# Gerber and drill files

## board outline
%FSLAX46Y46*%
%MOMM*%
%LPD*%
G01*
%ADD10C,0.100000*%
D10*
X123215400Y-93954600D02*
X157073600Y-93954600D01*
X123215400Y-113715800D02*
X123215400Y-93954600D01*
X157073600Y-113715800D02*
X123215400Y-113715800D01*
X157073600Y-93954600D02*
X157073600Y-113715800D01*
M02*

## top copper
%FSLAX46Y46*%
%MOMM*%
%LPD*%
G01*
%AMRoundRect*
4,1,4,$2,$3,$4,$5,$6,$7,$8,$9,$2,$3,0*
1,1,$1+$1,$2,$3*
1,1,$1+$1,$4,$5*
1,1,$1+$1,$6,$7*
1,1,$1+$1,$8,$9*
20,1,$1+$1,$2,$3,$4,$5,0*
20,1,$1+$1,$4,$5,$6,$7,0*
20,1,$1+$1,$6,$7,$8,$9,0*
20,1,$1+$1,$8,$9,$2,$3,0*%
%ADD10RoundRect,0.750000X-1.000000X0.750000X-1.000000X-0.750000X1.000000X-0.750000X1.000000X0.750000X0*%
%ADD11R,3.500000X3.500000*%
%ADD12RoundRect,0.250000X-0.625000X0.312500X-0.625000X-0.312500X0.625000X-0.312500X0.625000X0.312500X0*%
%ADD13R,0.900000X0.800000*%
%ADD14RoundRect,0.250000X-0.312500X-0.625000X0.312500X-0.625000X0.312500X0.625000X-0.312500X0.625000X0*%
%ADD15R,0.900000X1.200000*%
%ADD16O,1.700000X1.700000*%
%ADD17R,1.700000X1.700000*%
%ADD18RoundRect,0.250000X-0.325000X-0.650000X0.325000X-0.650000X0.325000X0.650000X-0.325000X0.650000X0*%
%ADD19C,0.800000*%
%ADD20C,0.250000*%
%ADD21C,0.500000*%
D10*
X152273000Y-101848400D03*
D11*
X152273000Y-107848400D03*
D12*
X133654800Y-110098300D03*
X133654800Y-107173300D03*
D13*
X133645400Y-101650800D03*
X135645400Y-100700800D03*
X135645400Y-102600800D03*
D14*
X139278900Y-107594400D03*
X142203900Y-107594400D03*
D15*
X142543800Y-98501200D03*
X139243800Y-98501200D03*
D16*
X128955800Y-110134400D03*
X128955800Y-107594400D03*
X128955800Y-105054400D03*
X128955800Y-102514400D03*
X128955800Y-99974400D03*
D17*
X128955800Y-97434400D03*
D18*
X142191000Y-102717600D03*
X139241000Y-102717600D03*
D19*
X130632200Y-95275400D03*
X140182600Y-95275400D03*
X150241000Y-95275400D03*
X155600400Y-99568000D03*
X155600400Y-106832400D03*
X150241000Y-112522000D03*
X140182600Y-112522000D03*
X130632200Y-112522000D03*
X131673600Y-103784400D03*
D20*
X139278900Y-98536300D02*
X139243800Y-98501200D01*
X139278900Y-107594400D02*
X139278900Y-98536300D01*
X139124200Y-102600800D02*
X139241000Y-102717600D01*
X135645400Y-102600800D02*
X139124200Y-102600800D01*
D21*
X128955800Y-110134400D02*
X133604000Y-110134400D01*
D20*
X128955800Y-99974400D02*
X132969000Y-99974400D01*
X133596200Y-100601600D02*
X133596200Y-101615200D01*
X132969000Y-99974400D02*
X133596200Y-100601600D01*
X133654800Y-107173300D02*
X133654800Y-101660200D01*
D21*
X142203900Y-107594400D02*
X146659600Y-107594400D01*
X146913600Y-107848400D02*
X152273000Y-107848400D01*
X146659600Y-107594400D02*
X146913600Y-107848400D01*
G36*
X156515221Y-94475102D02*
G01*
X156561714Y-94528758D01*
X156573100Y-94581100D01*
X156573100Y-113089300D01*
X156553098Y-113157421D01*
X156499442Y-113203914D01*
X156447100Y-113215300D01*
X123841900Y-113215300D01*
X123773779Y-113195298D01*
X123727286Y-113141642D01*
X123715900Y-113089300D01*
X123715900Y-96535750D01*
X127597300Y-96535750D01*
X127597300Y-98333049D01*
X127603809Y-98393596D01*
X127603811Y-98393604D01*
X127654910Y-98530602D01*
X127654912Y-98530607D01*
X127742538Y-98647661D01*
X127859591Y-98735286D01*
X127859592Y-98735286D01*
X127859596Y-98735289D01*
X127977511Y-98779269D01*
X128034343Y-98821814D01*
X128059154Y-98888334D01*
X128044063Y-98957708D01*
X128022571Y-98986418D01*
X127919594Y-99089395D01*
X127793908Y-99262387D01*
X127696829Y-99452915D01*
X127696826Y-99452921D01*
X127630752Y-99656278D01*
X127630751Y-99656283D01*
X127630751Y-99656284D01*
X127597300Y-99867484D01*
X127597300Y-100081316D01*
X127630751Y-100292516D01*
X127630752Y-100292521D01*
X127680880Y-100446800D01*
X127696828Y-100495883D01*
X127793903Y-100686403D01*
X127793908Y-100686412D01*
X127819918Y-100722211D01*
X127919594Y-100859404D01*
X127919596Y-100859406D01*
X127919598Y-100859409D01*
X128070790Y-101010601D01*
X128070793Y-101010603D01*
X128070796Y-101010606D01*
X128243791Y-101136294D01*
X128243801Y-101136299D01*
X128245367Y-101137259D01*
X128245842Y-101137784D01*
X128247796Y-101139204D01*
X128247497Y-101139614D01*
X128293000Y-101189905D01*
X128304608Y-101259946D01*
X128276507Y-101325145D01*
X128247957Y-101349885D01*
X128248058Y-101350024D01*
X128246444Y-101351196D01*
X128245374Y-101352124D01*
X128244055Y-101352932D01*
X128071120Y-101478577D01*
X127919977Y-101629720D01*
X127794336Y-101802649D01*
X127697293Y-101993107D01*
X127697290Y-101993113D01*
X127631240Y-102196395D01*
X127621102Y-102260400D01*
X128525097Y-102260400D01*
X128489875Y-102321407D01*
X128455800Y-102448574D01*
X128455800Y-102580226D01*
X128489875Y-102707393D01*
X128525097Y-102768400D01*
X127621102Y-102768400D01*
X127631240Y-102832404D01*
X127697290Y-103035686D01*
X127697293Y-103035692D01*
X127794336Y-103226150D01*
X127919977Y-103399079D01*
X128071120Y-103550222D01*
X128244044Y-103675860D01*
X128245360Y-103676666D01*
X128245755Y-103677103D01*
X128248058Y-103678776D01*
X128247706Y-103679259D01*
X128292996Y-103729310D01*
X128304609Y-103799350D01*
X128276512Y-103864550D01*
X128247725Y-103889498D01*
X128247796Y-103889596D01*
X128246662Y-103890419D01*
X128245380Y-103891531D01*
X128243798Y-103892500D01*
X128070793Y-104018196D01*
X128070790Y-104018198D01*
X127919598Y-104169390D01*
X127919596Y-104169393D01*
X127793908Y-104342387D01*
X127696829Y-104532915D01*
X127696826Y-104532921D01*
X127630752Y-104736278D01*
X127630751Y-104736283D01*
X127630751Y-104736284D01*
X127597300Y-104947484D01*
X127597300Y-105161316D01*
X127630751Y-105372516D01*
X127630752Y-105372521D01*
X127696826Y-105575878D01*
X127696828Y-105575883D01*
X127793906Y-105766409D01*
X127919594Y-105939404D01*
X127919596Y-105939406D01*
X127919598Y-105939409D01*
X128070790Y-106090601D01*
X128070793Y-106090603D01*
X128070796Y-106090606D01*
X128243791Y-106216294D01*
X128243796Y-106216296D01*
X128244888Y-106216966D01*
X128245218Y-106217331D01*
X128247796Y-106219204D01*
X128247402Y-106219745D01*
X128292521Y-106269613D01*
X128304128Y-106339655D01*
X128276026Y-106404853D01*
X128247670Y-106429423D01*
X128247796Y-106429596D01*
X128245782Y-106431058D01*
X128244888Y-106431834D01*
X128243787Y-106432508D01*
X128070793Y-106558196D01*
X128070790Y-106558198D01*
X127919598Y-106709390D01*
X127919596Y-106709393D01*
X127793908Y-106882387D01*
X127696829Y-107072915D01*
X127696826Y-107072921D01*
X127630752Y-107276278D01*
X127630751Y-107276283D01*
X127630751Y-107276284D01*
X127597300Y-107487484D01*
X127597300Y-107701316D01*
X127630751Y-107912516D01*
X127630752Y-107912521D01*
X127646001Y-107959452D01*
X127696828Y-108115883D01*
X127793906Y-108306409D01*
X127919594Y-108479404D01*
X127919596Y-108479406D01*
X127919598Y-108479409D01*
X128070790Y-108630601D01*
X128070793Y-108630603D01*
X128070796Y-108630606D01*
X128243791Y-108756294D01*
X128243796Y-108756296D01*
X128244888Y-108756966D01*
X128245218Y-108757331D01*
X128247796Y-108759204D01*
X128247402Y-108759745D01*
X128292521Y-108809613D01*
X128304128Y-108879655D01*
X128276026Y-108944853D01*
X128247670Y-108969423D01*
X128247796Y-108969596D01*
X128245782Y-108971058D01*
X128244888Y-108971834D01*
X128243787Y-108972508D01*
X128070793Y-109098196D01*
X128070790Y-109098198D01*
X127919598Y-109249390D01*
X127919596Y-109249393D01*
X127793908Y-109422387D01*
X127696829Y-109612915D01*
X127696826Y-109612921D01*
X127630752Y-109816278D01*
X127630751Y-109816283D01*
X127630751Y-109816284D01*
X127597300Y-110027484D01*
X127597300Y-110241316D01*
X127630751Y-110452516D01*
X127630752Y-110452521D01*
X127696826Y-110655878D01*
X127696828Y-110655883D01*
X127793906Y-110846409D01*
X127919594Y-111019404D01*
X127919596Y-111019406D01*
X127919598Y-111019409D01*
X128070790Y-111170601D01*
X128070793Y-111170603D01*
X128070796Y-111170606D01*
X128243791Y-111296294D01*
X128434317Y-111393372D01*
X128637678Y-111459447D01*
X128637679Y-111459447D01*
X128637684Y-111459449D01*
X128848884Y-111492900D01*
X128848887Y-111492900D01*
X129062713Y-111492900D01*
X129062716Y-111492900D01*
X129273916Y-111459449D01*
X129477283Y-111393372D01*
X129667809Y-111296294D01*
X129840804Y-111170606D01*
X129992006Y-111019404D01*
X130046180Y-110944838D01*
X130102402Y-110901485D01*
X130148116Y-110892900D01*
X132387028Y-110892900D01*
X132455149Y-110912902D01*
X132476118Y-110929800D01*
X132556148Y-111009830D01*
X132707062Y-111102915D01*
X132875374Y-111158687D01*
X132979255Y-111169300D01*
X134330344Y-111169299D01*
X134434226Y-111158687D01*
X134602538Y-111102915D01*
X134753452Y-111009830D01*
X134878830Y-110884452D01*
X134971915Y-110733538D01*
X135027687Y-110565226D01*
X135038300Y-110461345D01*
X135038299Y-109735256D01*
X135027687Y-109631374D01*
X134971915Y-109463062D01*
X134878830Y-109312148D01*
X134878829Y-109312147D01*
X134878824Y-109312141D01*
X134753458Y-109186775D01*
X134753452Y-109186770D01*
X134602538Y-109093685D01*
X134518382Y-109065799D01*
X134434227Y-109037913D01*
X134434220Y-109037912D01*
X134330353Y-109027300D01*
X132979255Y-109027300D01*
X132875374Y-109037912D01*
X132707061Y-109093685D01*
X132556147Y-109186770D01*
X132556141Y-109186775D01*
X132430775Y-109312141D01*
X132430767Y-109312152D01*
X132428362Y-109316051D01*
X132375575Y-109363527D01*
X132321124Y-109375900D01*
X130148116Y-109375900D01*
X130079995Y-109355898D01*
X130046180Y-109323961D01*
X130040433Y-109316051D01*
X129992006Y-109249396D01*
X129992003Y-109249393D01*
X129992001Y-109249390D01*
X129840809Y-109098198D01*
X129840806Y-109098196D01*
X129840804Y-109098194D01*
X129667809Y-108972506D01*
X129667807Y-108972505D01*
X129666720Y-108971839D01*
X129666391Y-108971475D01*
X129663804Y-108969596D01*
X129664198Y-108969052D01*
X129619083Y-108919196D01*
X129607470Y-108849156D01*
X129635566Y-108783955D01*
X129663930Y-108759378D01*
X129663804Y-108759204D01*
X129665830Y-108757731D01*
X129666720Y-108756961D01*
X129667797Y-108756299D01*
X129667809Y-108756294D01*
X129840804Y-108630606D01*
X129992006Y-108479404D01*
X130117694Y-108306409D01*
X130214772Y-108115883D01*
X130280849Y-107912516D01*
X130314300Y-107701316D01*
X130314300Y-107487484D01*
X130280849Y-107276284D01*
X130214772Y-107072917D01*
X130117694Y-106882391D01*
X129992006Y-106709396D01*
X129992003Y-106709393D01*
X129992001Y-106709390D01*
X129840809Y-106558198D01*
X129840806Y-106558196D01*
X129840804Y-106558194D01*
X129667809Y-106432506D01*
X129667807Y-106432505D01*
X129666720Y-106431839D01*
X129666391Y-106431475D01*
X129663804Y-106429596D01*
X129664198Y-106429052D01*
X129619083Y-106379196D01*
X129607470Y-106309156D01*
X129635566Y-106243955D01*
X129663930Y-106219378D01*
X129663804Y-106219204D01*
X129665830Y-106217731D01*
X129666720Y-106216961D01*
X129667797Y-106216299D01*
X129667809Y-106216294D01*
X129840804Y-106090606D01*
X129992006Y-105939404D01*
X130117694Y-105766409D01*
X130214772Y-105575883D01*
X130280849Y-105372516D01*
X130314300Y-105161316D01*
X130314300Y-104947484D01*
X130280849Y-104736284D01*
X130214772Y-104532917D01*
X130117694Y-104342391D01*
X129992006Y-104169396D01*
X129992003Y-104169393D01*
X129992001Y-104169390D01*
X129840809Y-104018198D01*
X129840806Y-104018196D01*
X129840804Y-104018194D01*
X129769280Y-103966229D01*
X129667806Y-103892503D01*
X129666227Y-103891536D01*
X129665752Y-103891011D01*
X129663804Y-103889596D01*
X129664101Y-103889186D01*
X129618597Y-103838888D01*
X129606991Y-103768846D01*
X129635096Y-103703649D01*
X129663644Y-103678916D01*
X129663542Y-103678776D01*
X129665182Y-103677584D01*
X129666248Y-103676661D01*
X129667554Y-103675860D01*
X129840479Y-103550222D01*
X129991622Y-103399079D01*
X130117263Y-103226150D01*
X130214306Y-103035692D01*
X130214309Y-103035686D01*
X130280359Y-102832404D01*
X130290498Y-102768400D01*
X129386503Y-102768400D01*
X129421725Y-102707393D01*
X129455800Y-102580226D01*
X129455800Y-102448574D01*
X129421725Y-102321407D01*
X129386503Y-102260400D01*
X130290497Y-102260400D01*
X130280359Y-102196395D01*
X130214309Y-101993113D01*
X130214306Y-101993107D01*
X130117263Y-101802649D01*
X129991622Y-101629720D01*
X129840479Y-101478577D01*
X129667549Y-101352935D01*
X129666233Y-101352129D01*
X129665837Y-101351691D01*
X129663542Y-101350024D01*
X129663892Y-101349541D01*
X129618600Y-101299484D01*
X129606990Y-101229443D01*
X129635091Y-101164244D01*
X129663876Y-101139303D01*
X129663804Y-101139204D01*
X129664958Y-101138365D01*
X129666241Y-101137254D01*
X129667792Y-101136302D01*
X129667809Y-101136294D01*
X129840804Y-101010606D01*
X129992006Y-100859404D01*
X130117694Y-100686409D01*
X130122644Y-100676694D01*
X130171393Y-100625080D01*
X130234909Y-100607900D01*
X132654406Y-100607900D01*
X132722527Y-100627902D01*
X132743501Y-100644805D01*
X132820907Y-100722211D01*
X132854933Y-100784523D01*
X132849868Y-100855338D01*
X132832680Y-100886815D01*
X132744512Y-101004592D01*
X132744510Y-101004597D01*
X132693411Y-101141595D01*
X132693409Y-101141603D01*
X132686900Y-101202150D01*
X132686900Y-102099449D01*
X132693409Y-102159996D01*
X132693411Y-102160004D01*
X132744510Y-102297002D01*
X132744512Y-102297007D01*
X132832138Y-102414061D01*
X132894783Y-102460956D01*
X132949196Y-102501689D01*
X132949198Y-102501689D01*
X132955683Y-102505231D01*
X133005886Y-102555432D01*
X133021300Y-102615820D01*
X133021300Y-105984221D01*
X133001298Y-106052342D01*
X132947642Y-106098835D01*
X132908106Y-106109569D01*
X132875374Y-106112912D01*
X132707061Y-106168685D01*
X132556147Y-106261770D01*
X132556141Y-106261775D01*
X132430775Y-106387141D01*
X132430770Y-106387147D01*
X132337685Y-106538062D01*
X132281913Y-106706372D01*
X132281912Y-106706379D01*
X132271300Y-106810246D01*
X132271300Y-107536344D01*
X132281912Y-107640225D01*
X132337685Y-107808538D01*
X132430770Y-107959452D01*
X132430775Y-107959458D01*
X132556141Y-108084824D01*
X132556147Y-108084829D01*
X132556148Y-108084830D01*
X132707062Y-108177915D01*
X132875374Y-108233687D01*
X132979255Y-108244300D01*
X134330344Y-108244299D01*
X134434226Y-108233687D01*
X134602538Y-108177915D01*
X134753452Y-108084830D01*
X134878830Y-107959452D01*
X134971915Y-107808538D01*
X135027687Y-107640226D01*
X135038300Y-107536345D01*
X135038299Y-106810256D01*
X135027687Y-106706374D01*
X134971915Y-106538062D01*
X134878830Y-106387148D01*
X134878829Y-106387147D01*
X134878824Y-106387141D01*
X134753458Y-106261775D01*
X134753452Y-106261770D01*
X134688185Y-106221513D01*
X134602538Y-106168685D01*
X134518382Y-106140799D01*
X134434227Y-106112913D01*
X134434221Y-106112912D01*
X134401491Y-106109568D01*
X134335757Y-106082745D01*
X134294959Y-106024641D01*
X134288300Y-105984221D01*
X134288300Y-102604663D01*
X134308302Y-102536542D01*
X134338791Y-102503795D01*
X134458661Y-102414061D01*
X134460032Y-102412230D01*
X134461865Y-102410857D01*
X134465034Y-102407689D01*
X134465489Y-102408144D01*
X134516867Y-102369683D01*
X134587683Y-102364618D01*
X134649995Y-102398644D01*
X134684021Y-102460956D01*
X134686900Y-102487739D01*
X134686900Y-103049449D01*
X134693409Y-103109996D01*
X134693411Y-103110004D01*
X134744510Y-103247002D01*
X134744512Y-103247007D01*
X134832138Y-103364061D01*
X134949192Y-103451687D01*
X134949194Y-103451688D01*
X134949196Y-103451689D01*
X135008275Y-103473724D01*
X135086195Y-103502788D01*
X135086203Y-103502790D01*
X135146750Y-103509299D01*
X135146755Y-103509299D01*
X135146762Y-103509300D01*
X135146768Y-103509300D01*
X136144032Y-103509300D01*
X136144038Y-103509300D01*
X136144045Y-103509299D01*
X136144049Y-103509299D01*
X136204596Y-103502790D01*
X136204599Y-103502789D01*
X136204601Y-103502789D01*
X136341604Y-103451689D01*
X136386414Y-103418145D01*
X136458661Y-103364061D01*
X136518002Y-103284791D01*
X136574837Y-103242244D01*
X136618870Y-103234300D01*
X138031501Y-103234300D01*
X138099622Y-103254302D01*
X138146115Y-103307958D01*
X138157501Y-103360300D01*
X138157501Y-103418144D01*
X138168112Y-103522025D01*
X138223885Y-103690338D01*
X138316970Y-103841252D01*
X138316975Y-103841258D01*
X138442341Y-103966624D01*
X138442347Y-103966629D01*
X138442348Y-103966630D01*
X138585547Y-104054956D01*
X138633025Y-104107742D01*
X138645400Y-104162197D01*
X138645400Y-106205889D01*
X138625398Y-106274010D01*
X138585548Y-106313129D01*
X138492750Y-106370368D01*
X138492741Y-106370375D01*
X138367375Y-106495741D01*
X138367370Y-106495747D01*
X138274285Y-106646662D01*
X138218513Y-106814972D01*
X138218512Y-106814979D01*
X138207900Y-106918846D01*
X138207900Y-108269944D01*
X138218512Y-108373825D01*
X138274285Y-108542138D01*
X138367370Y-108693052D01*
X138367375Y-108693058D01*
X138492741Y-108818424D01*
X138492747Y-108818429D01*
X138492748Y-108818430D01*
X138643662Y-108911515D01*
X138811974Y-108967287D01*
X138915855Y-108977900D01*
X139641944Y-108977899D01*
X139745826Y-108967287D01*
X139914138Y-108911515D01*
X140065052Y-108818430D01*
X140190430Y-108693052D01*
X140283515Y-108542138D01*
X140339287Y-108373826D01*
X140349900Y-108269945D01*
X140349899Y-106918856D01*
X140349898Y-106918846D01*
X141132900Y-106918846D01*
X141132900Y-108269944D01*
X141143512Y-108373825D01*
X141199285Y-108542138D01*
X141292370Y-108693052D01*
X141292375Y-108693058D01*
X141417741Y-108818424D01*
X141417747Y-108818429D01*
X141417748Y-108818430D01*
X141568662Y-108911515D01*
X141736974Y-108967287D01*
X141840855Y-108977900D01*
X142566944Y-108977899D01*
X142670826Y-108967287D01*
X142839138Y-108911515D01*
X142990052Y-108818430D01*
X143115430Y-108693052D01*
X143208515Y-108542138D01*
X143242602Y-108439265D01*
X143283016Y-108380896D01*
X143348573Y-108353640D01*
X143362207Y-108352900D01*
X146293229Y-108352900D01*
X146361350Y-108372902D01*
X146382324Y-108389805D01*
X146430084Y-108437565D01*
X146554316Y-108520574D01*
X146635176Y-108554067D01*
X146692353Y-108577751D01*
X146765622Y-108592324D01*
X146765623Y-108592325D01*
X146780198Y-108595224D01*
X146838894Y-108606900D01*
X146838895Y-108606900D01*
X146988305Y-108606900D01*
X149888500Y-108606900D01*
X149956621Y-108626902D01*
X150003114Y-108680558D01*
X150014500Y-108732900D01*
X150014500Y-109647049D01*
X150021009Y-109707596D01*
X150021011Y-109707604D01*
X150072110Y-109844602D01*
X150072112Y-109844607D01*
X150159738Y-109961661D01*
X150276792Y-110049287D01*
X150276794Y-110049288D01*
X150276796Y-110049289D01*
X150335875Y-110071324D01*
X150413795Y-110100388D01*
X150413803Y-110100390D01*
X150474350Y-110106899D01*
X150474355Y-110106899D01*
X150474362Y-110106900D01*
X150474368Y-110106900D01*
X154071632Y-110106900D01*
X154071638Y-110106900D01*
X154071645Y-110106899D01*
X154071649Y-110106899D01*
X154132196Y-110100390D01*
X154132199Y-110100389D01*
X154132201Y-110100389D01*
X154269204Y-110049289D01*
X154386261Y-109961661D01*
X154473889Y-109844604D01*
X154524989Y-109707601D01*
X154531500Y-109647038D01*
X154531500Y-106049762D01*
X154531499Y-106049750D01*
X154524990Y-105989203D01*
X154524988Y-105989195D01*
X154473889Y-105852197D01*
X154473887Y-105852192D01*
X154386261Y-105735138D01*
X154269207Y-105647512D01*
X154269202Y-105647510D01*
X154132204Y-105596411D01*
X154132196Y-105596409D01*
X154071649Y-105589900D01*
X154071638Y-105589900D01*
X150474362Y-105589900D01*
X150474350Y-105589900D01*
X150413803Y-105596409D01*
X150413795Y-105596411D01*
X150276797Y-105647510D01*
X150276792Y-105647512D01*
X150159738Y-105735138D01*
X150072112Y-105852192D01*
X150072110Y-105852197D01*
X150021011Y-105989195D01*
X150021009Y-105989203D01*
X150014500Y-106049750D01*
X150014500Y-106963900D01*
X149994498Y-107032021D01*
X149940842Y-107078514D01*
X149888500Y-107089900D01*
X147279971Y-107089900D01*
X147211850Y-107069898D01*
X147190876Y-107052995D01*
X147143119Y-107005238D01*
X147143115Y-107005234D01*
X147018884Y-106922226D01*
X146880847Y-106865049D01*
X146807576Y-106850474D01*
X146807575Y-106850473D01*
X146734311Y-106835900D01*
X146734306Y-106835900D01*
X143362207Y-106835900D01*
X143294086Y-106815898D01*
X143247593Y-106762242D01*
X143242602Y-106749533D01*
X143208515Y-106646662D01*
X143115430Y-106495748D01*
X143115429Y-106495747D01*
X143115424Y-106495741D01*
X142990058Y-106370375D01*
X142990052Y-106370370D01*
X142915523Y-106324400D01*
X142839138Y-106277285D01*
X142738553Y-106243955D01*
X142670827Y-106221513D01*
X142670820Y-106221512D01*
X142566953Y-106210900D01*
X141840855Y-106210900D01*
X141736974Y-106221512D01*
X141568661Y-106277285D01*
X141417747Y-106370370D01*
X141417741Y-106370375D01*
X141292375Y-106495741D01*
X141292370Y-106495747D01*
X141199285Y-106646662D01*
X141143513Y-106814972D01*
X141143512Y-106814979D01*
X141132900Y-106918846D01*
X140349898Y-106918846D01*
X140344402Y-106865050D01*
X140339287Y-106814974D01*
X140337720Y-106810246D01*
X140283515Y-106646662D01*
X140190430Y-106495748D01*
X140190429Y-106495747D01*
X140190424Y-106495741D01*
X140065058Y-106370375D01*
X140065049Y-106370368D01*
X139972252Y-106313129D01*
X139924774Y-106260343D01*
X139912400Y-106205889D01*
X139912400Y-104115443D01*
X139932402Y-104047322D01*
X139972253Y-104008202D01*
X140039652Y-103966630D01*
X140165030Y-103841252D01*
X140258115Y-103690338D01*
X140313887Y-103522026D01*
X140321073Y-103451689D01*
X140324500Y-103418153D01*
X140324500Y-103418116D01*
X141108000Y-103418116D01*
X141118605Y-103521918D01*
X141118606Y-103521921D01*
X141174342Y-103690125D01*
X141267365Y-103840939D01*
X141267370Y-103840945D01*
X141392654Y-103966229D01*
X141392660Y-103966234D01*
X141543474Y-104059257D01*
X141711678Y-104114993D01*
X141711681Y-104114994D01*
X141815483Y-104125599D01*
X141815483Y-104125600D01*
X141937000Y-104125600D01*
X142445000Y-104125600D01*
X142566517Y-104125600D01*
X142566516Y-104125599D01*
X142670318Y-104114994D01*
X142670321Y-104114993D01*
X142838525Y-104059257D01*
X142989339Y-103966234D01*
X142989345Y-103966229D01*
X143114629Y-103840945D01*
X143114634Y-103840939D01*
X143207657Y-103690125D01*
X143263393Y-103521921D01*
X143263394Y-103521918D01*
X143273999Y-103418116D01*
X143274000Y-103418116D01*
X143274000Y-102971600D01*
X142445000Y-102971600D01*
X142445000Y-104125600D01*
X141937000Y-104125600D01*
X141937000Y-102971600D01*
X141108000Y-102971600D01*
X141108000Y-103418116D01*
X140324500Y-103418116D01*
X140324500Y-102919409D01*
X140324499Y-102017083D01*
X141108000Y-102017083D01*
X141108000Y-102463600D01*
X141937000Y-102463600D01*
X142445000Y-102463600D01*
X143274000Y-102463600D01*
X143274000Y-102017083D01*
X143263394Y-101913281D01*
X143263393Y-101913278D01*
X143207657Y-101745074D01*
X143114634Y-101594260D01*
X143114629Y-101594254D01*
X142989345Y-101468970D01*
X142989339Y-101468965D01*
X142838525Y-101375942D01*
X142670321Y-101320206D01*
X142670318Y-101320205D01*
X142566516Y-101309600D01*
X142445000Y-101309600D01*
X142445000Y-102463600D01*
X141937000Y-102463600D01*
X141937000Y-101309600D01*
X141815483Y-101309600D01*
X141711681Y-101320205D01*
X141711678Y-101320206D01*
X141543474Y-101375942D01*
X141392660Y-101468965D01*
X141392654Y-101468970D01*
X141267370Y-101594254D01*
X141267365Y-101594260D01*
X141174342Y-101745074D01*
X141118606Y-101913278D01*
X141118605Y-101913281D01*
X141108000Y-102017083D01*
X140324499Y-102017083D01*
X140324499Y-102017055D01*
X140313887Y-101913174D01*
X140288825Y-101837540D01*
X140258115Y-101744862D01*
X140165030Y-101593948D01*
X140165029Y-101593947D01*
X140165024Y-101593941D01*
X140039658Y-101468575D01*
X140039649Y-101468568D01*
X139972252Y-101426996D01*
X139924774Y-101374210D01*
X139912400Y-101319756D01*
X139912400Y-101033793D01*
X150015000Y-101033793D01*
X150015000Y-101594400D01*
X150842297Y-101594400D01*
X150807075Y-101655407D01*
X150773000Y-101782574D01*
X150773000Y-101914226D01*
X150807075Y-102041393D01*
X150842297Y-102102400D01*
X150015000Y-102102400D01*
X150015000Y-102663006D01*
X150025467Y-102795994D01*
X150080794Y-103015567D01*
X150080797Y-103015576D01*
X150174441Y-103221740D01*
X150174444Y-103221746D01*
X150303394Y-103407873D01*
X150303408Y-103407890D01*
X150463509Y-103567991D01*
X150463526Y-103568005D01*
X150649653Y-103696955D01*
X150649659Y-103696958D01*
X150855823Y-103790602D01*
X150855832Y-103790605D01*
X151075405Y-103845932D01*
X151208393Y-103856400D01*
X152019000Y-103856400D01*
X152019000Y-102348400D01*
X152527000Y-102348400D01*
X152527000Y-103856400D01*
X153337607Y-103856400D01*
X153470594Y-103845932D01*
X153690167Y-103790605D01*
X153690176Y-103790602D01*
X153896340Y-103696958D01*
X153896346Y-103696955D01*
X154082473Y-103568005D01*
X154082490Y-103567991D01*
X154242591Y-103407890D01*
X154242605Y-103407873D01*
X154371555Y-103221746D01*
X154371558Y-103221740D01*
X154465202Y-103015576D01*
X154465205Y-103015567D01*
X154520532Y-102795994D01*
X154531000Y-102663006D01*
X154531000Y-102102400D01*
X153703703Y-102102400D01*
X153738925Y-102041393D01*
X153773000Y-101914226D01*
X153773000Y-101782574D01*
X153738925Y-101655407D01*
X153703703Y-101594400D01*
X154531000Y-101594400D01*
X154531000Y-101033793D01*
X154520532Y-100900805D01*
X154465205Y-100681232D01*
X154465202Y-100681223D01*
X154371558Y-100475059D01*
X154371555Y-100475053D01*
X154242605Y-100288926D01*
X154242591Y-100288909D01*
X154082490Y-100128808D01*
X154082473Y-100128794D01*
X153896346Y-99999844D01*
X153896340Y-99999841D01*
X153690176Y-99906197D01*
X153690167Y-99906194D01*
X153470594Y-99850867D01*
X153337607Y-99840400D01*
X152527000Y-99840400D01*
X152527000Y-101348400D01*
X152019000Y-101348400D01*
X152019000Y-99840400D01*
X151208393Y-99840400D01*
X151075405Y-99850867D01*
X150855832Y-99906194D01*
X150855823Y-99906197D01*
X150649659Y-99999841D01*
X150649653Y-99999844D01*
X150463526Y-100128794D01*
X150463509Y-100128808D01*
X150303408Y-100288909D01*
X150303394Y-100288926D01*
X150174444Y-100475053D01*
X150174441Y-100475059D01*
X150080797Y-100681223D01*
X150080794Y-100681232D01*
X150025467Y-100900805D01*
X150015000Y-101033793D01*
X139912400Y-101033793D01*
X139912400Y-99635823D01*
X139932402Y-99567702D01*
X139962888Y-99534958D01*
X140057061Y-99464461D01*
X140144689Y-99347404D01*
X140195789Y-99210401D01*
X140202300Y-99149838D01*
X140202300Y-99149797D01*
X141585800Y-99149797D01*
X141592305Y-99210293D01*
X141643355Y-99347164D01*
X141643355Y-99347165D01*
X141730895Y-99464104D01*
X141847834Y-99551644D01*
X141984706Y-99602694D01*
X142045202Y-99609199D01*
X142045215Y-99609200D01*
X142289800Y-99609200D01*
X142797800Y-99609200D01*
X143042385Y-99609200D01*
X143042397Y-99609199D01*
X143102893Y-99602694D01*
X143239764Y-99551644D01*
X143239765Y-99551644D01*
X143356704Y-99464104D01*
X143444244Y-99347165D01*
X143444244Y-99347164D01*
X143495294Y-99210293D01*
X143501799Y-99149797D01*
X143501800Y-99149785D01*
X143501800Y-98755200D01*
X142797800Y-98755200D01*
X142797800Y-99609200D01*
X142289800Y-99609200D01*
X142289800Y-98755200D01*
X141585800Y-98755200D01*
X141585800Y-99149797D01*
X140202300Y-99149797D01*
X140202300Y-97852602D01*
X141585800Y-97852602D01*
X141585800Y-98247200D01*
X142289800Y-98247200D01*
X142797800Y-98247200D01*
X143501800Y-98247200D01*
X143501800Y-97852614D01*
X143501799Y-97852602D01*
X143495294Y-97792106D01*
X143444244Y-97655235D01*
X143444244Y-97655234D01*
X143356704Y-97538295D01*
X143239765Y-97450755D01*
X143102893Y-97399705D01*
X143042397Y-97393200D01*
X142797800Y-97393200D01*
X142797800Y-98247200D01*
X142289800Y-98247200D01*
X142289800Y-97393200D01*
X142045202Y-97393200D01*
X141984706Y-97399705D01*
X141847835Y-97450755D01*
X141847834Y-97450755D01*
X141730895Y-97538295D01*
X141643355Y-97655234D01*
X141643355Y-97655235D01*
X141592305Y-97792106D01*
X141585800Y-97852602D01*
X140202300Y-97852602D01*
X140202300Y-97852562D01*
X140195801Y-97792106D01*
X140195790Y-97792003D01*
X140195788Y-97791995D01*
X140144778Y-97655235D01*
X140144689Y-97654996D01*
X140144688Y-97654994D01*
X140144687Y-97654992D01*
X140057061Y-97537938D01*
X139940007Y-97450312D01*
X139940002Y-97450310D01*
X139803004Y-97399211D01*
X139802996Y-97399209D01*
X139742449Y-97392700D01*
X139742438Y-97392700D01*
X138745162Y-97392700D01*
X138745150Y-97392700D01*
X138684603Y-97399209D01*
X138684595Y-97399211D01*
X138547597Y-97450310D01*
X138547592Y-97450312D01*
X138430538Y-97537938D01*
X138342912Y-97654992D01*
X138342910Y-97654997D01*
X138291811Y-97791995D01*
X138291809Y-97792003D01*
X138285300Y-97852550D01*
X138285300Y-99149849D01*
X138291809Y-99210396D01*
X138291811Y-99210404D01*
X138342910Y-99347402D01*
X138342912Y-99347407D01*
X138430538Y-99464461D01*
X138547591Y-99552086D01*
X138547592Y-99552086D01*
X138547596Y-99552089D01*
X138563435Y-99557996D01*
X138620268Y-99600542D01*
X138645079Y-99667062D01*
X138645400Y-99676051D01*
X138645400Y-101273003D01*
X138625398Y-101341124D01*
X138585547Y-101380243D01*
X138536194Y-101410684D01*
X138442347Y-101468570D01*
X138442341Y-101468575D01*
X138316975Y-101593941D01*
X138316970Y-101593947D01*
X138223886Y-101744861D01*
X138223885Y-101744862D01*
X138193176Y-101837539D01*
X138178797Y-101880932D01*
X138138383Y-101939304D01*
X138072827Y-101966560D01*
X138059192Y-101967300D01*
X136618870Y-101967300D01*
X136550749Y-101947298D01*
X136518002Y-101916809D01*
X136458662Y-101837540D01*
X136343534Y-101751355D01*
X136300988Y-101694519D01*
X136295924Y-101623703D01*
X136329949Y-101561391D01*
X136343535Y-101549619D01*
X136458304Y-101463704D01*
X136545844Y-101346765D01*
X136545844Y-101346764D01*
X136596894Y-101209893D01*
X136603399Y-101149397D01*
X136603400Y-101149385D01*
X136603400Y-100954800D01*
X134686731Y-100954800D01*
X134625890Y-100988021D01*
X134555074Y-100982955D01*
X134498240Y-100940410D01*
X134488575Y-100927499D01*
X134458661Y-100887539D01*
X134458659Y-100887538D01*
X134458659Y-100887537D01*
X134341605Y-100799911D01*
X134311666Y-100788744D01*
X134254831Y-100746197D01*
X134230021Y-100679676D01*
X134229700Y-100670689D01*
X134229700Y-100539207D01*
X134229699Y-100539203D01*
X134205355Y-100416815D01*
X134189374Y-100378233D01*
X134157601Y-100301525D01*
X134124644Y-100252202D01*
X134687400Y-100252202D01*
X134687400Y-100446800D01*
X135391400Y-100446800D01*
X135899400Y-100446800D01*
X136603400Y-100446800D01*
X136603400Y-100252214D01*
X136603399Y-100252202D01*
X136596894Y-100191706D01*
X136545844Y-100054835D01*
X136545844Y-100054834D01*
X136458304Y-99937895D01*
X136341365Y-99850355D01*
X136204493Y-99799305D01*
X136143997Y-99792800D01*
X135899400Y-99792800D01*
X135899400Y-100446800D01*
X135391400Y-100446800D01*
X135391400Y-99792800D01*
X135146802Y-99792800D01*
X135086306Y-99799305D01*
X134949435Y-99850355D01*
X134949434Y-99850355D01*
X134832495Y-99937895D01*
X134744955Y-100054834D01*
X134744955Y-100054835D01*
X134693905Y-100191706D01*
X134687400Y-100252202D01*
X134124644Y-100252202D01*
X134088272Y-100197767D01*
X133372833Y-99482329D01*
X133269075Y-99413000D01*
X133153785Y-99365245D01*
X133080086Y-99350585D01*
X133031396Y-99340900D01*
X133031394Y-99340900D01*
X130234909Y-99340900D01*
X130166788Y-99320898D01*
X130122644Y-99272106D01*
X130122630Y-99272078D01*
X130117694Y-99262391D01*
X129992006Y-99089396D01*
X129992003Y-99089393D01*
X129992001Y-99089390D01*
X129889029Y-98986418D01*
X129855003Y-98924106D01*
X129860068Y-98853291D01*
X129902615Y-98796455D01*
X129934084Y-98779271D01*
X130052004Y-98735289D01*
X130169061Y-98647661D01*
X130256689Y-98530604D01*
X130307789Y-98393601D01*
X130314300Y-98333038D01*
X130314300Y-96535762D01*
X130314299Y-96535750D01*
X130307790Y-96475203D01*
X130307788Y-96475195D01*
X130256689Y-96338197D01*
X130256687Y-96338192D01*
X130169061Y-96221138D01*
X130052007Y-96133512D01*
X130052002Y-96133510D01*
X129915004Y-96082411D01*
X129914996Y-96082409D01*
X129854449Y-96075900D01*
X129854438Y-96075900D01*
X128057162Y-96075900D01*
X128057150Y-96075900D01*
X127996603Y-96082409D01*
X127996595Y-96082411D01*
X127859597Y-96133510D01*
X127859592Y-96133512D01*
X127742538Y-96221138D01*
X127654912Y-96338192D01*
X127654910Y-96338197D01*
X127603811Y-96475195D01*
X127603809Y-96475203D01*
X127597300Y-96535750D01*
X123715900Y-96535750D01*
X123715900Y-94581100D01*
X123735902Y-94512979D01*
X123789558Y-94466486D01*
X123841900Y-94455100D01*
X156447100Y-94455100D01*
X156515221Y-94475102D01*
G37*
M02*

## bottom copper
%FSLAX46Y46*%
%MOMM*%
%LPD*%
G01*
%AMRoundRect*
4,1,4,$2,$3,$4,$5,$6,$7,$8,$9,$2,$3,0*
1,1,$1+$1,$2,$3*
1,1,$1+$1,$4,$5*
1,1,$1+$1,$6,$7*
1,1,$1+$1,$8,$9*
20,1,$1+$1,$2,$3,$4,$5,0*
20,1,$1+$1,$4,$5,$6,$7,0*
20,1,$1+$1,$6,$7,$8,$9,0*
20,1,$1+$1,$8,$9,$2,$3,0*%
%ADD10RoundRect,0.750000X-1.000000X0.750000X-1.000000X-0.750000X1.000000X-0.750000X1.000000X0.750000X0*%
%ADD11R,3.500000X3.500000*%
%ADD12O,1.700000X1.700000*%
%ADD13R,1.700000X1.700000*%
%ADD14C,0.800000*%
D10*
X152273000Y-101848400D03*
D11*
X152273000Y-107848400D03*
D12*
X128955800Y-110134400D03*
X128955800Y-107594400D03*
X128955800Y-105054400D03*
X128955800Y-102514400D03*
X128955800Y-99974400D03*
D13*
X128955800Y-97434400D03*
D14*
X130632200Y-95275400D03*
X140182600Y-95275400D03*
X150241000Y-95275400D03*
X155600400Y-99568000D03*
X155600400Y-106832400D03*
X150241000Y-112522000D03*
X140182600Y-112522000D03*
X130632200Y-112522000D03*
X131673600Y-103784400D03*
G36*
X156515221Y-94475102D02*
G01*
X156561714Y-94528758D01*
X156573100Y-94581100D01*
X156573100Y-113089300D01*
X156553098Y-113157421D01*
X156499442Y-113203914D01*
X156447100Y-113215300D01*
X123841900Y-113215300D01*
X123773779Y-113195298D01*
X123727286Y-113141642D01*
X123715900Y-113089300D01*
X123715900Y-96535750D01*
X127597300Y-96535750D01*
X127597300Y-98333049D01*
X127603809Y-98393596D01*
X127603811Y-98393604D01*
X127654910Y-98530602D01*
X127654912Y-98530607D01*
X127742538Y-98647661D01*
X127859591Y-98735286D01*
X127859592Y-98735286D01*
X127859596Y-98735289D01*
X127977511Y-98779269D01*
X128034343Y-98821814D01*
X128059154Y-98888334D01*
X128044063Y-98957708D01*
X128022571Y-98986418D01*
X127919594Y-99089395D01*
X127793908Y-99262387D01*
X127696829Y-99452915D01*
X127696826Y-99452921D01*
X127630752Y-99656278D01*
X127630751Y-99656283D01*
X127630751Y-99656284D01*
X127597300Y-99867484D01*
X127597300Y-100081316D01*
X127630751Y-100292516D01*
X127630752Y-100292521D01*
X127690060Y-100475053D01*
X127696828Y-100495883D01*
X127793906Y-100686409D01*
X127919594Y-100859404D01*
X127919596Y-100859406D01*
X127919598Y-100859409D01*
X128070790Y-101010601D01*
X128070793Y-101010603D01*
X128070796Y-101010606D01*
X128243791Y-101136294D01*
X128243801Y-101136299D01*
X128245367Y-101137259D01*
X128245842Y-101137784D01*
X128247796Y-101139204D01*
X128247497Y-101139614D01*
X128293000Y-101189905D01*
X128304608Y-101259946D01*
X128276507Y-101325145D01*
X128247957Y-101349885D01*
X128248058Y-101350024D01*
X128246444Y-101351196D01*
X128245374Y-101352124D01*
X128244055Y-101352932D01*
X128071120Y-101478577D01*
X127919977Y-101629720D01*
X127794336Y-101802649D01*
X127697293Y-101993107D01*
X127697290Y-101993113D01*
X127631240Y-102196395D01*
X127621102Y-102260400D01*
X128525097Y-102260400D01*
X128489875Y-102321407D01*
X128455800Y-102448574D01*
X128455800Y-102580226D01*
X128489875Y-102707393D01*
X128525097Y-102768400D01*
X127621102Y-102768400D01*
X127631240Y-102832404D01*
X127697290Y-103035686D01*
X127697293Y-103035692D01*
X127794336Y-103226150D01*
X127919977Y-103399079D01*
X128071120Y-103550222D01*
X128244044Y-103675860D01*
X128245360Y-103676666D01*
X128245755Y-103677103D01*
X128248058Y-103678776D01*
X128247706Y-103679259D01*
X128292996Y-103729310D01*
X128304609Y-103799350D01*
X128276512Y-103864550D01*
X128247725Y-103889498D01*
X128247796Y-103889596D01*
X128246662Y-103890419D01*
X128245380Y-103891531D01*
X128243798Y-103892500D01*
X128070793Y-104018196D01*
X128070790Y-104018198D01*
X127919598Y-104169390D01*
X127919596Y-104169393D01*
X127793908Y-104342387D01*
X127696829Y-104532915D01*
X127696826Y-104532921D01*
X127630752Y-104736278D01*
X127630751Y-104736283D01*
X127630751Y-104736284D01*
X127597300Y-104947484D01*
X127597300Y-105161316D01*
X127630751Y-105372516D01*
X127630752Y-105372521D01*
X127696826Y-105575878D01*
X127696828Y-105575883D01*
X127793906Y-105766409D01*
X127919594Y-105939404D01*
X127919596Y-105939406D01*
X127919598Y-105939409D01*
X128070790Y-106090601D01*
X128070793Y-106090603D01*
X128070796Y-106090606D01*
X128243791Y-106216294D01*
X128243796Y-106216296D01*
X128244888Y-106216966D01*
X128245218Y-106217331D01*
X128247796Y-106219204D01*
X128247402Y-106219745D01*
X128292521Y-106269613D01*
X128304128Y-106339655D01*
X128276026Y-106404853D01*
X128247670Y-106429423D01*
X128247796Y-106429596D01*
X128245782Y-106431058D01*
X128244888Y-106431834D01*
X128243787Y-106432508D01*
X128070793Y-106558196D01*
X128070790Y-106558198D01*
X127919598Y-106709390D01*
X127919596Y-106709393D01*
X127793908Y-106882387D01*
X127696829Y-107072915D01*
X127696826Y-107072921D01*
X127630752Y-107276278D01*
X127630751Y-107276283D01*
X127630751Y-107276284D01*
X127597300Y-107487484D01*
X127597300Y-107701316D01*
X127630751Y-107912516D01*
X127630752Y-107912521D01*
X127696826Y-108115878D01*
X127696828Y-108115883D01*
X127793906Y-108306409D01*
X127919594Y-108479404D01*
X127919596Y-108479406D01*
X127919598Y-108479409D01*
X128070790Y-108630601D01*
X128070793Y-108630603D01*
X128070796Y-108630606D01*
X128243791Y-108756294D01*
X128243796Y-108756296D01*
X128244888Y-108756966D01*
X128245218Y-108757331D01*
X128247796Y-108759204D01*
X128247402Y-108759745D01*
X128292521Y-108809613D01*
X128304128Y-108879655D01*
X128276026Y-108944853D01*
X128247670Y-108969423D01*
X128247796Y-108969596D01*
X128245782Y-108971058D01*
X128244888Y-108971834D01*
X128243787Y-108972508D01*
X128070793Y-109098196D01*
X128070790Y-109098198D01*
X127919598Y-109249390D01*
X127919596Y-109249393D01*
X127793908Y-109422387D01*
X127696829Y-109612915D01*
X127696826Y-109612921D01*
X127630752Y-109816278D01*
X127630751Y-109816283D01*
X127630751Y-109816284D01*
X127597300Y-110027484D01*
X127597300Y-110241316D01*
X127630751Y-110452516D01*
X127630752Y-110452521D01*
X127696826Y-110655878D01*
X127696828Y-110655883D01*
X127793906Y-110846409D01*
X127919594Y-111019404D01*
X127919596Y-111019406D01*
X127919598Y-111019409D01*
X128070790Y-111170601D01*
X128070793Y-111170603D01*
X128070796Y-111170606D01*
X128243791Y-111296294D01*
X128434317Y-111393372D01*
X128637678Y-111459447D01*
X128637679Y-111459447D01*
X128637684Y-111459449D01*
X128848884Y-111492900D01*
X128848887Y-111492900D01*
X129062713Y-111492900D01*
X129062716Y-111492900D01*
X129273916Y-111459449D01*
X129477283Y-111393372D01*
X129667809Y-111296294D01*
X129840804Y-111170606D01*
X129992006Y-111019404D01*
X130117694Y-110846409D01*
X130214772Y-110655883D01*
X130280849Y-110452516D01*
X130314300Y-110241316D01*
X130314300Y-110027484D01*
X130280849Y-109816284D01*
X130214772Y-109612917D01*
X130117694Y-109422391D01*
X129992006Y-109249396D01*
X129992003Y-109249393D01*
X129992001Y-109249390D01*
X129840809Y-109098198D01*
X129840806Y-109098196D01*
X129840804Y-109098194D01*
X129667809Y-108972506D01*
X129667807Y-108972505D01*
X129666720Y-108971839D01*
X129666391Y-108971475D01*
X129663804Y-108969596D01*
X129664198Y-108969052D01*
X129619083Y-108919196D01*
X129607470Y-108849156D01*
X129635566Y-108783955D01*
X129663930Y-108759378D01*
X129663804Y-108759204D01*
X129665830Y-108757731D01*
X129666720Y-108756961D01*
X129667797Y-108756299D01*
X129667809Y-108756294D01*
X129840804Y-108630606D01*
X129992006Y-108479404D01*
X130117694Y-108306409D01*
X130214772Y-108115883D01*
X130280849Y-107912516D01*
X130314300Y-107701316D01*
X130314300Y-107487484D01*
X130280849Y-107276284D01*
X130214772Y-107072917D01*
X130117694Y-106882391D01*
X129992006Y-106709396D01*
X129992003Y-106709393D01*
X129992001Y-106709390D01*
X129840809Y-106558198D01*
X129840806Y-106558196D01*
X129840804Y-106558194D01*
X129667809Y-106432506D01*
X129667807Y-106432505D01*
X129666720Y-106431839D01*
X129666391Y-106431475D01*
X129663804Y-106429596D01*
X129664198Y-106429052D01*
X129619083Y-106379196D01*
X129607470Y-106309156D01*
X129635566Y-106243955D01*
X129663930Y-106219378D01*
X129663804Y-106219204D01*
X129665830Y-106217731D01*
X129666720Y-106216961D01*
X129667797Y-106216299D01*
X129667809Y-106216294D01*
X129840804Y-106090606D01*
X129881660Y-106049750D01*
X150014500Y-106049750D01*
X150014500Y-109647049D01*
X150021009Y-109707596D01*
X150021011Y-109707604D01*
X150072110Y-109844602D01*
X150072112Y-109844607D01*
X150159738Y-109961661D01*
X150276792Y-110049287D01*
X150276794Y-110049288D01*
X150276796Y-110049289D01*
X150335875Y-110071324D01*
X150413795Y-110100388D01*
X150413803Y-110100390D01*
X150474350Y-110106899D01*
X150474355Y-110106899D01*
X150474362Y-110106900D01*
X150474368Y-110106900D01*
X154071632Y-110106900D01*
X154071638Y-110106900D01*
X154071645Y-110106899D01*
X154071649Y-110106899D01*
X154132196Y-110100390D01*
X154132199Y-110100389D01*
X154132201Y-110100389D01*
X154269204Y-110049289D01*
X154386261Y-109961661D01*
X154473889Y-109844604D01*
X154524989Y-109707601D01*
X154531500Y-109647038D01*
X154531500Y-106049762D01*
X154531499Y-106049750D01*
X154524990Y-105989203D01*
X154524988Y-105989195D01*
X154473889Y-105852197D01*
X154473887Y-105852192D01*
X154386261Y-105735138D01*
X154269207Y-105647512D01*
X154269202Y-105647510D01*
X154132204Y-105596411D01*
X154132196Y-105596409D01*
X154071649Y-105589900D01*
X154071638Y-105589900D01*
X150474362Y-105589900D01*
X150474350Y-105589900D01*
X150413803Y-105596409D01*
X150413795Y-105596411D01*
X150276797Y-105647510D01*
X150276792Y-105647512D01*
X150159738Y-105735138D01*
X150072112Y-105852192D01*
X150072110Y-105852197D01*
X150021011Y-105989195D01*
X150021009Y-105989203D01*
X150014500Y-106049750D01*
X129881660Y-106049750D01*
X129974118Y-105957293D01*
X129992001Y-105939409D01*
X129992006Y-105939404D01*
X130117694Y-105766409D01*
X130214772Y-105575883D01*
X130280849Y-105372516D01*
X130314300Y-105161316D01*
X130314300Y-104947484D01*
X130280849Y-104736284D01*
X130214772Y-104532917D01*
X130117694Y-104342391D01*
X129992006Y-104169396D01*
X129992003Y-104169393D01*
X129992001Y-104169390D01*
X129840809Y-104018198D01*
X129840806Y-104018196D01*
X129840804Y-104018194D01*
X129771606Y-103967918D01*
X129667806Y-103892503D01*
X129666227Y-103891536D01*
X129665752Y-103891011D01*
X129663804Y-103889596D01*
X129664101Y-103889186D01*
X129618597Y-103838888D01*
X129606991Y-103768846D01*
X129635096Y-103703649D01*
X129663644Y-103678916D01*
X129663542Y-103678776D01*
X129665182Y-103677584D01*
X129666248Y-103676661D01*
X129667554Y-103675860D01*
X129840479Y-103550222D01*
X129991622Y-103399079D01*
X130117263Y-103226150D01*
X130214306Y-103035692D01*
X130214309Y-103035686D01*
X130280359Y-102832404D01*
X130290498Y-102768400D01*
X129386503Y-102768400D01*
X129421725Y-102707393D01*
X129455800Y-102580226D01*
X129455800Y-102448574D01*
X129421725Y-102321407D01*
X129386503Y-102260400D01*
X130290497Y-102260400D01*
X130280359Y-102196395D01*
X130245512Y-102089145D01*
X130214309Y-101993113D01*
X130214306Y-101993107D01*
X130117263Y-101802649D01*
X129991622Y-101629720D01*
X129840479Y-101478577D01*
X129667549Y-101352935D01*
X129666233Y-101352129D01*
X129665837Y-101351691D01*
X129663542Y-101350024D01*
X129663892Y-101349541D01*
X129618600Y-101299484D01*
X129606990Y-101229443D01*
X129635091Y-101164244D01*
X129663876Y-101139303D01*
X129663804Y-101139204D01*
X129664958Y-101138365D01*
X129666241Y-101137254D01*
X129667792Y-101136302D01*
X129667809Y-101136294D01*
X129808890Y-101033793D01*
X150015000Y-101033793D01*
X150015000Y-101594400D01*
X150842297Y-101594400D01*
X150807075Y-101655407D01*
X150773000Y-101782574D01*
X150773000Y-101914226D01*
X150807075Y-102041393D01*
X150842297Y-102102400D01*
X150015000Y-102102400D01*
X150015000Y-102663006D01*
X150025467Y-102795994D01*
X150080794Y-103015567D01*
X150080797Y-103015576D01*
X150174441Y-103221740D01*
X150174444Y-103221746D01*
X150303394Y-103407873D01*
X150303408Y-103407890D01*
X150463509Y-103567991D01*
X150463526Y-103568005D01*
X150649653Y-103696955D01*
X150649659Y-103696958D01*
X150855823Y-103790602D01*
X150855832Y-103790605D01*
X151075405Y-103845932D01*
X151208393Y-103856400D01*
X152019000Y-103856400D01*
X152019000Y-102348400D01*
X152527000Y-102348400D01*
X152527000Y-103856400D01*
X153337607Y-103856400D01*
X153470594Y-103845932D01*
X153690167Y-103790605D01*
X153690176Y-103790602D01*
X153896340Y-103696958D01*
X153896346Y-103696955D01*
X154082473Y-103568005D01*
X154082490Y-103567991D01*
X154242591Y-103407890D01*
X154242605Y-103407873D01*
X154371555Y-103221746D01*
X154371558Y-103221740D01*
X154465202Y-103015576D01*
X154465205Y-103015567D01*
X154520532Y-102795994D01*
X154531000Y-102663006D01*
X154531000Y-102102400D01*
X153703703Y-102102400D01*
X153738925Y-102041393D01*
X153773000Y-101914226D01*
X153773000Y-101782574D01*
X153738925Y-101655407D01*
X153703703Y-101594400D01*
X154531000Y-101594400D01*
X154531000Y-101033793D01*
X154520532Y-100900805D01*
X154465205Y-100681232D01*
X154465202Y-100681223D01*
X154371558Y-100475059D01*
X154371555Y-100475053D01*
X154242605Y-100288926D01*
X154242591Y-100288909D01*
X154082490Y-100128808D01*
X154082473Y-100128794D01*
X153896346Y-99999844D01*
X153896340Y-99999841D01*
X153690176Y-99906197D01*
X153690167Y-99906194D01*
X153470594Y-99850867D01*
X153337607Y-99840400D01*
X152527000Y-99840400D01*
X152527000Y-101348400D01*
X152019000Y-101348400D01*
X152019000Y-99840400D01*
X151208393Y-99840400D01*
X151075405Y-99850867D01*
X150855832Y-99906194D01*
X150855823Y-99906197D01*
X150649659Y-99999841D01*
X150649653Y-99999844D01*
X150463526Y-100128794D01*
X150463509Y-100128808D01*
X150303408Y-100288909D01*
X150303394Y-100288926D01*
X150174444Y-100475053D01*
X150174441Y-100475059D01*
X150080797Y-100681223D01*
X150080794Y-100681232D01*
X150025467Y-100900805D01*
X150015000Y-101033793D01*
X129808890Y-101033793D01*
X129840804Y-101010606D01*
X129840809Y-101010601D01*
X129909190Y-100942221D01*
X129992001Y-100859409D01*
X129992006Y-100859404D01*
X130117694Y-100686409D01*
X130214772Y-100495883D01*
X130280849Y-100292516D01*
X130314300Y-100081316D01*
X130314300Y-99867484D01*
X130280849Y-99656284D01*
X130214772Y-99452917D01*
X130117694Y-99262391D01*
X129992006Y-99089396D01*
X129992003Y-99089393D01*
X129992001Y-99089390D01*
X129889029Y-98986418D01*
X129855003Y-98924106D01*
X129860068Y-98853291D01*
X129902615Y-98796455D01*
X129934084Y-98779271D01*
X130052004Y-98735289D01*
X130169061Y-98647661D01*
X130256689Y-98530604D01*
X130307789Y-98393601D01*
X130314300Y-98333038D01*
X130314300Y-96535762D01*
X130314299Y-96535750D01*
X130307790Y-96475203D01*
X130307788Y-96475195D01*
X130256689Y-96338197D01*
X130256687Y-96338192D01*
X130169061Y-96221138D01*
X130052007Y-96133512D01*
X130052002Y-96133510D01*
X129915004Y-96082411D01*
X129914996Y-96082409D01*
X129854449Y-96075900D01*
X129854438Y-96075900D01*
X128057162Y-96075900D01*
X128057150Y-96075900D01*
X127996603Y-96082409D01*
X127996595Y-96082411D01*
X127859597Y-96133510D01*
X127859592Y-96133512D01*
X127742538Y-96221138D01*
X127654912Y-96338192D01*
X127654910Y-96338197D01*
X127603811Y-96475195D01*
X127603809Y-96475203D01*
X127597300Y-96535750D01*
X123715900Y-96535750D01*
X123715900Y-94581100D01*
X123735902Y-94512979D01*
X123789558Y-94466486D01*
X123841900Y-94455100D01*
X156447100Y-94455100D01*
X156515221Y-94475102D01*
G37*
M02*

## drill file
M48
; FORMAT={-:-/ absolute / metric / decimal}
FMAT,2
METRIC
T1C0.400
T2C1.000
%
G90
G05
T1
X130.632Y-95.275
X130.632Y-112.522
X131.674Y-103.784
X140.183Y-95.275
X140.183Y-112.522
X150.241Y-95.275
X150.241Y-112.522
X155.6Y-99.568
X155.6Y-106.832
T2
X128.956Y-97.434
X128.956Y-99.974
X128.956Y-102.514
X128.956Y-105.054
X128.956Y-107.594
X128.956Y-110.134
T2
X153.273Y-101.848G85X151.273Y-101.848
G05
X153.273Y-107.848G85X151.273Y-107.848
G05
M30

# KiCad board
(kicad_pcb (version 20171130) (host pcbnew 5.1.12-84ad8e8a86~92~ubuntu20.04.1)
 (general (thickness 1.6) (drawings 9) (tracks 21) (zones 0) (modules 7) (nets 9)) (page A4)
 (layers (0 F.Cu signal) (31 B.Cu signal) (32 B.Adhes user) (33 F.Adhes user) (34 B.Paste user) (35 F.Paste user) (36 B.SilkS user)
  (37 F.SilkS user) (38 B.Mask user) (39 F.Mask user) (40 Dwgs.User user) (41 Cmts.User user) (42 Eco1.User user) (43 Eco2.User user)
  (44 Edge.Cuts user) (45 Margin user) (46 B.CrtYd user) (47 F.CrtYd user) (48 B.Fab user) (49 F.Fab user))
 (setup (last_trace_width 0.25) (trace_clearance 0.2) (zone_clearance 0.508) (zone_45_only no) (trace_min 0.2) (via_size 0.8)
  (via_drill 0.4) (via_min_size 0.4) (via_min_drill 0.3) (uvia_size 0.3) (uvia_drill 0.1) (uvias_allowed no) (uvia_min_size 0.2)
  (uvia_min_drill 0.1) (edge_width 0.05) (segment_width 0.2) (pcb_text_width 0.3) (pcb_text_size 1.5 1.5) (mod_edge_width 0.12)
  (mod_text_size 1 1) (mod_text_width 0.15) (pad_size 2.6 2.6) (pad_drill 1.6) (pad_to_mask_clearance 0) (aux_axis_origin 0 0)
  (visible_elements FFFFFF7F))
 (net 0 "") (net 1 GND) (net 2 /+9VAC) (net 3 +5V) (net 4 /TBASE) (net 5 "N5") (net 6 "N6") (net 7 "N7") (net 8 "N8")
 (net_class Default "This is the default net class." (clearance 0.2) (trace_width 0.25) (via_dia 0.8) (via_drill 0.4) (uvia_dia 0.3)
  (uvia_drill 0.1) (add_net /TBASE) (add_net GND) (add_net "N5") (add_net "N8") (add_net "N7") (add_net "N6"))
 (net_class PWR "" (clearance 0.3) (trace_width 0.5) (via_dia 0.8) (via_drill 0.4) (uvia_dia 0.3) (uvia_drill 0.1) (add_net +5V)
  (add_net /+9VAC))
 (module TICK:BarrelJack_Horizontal (layer F.Cu) (at 152.273 107.8484 270)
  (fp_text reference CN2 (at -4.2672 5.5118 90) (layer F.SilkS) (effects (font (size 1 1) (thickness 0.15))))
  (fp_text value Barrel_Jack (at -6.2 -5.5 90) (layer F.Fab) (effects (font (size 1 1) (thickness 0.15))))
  (pad 2 thru_hole roundrect (at -6 0 270) (size 3 3.5) (drill oval 1 3) (layers *.Cu *.Mask) (roundrect_rratio 0.25) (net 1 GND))
  (pad 1 thru_hole rect (at 0 0 270) (size 3.5 3.5) (drill oval 1 3) (layers *.Cu *.Mask) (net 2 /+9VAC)))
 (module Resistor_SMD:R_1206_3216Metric (layer F.Cu) (at 133.6548 108.6358 270)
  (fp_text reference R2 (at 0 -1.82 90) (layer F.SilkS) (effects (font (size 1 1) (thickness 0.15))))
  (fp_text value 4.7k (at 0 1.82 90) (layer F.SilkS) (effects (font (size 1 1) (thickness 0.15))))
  (pad 2 smd roundrect (at 1.4625 0 270) (size 1.125 1.75) (layers F.Cu F.Paste F.Mask) (roundrect_rratio 0.222222) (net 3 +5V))
  (pad 1 smd roundrect (at -1.4625 0 270) (size 1.125 1.75) (layers F.Cu F.Paste F.Mask) (roundrect_rratio 0.222222) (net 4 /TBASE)))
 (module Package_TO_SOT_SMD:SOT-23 (layer F.Cu) (at 134.6454 101.6508 180)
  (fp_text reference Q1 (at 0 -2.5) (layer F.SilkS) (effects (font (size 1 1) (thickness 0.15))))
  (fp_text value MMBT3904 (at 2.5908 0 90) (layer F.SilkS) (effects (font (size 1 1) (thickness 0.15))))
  (pad 3 smd rect (at 1 0 180) (size 0.9 0.8) (layers F.Cu F.Paste F.Mask) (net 4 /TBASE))
  (pad 2 smd rect (at -1 0.95 180) (size 0.9 0.8) (layers F.Cu F.Paste F.Mask) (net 1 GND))
  (pad 1 smd rect (at -1 -0.95 180) (size 0.9 0.8) (layers F.Cu F.Paste F.Mask) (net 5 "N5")))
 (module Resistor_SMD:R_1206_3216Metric (layer F.Cu) (at 140.7414 107.5944)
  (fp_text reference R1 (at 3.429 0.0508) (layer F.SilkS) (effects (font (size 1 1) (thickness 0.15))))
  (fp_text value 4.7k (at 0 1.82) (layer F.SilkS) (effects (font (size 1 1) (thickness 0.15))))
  (pad 1 smd roundrect (at -1.4625 0) (size 1.125 1.75) (layers F.Cu F.Paste F.Mask) (roundrect_rratio 0.222222) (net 5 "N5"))
  (pad 2 smd roundrect (at 1.4625 0) (size 1.125 1.75) (layers F.Cu F.Paste F.Mask) (roundrect_rratio 0.222222) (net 2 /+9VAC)))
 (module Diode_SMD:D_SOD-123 (layer F.Cu) (at 140.8938 98.5012)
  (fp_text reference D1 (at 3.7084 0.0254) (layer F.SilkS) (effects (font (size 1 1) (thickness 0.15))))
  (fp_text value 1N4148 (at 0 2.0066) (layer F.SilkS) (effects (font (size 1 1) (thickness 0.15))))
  (pad 2 smd rect (at 1.65 0) (size 0.9 1.2) (layers F.Cu F.Paste F.Mask) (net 1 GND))
  (pad 1 smd rect (at -1.65 0) (size 0.9 1.2) (layers F.Cu F.Paste F.Mask) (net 5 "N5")))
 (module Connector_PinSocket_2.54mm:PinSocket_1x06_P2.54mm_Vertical (layer F.Cu) (at 128.9558 97.4344)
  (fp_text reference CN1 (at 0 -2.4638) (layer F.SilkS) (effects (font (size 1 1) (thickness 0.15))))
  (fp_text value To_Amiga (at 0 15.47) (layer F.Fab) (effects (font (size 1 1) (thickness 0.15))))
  (pad 6 thru_hole oval (at 0 12.7) (size 1.7 1.7) (drill 1) (layers *.Cu *.Mask) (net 3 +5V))
  (pad 5 thru_hole oval (at 0 10.16) (size 1.7 1.7) (drill 1) (layers *.Cu *.Mask) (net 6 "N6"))
  (pad 4 thru_hole oval (at 0 7.62) (size 1.7 1.7) (drill 1) (layers *.Cu *.Mask) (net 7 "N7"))
  (pad 3 thru_hole oval (at 0 5.08) (size 1.7 1.7) (drill 1) (layers *.Cu *.Mask) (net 1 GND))
  (pad 2 thru_hole oval (at 0 2.54) (size 1.7 1.7) (drill 1) (layers *.Cu *.Mask) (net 4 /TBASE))
  (pad 1 thru_hole rect (at 0 0) (size 1.7 1.7) (drill 1) (layers *.Cu *.Mask) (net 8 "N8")))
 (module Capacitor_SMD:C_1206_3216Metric (layer F.Cu) (at 140.716 102.7176)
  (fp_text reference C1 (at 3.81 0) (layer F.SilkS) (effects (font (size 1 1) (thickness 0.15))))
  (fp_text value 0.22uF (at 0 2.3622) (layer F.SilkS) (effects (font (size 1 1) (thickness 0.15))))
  (pad 2 smd roundrect (at 1.475 0) (size 1.15 1.8) (layers F.Cu F.Paste F.Mask) (roundrect_rratio 0.217391) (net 1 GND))
  (pad 1 smd roundrect (at -1.475 0) (size 1.15 1.8) (layers F.Cu F.Paste F.Mask) (roundrect_rratio 0.217391) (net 5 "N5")))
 (gr_line (start 123.2154 93.9546) (end 157.0736 93.9546) (layer Edge.Cuts) (width 0.1))
 (gr_line (start 123.2154 113.7158) (end 123.2154 93.9546) (layer Edge.Cuts) (width 0.1))
 (gr_line (start 157.0736 113.7158) (end 123.2154 113.7158) (layer Edge.Cuts) (width 0.1))
 (gr_line (start 157.0736 93.9546) (end 157.0736 113.7158) (layer Edge.Cuts) (width 0.1))
 (via (at 130.6322 95.2754) (size 0.8) (drill 0.4) (layers F.Cu B.Cu) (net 1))
 (via (at 140.1826 95.2754) (size 0.8) (drill 0.4) (layers F.Cu B.Cu) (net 1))
 (via (at 150.241 95.2754) (size 0.8) (drill 0.4) (layers F.Cu B.Cu) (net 1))
 (via (at 155.6004 99.568) (size 0.8) (drill 0.4) (layers F.Cu B.Cu) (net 1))
 (via (at 155.6004 106.8324) (size 0.8) (drill 0.4) (layers F.Cu B.Cu) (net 1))
 (via (at 150.241 112.522) (size 0.8) (drill 0.4) (layers F.Cu B.Cu) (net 1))
 (via (at 140.1826 112.522) (size 0.8) (drill 0.4) (layers F.Cu B.Cu) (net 1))
 (via (at 130.6322 112.522) (size 0.8) (drill 0.4) (layers F.Cu B.Cu) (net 1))
 (via (at 131.6736 103.7844) (size 0.8) (drill 0.4) (layers F.Cu B.Cu) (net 1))
 (segment (start 139.2789 98.5363) (end 139.2438 98.5012) (width 0.25) (layer F.Cu) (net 5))
 (segment (start 139.2789 107.5944) (end 139.2789 98.5363) (width 0.25) (layer F.Cu) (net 5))
 (segment (start 139.1242 102.6008) (end 139.241 102.7176) (width 0.25) (layer F.Cu) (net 5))
 (segment (start 135.6454 102.6008) (end 139.1242 102.6008) (width 0.25) (layer F.Cu) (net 5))
 (segment (start 128.9558 110.1344) (end 133.604 110.1344) (width 0.5) (layer F.Cu) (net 3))
 (segment (start 128.9558 99.9744) (end 132.969 99.9744) (width 0.25) (layer F.Cu) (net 4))
 (segment (start 133.5962 100.6016) (end 133.5962 101.6152) (width 0.25) (layer F.Cu) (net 4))
 (segment (start 132.969 99.9744) (end 133.5962 100.6016) (width 0.25) (layer F.Cu) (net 4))
 (segment (start 133.6548 107.1733) (end 133.6548 101.6602) (width 0.25) (layer F.Cu) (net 4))
 (segment (start 142.2039 107.5944) (end 146.6596 107.5944) (width 0.5) (layer F.Cu) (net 2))
 (segment (start 146.9136 107.8484) (end 152.273 107.8484) (width 0.5) (layer F.Cu) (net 2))
 (segment (start 146.6596 107.5944) (end 146.9136 107.8484) (width 0.5) (layer F.Cu) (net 2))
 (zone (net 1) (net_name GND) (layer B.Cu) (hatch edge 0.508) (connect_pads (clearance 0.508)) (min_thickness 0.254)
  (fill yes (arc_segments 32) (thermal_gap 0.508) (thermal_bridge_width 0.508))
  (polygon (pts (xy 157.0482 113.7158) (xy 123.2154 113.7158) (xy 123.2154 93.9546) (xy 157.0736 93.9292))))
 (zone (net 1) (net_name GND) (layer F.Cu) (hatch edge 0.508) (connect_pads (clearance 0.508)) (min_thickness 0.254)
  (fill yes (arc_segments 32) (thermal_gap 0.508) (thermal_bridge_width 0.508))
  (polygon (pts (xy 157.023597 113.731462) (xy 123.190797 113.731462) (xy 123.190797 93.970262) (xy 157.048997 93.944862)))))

